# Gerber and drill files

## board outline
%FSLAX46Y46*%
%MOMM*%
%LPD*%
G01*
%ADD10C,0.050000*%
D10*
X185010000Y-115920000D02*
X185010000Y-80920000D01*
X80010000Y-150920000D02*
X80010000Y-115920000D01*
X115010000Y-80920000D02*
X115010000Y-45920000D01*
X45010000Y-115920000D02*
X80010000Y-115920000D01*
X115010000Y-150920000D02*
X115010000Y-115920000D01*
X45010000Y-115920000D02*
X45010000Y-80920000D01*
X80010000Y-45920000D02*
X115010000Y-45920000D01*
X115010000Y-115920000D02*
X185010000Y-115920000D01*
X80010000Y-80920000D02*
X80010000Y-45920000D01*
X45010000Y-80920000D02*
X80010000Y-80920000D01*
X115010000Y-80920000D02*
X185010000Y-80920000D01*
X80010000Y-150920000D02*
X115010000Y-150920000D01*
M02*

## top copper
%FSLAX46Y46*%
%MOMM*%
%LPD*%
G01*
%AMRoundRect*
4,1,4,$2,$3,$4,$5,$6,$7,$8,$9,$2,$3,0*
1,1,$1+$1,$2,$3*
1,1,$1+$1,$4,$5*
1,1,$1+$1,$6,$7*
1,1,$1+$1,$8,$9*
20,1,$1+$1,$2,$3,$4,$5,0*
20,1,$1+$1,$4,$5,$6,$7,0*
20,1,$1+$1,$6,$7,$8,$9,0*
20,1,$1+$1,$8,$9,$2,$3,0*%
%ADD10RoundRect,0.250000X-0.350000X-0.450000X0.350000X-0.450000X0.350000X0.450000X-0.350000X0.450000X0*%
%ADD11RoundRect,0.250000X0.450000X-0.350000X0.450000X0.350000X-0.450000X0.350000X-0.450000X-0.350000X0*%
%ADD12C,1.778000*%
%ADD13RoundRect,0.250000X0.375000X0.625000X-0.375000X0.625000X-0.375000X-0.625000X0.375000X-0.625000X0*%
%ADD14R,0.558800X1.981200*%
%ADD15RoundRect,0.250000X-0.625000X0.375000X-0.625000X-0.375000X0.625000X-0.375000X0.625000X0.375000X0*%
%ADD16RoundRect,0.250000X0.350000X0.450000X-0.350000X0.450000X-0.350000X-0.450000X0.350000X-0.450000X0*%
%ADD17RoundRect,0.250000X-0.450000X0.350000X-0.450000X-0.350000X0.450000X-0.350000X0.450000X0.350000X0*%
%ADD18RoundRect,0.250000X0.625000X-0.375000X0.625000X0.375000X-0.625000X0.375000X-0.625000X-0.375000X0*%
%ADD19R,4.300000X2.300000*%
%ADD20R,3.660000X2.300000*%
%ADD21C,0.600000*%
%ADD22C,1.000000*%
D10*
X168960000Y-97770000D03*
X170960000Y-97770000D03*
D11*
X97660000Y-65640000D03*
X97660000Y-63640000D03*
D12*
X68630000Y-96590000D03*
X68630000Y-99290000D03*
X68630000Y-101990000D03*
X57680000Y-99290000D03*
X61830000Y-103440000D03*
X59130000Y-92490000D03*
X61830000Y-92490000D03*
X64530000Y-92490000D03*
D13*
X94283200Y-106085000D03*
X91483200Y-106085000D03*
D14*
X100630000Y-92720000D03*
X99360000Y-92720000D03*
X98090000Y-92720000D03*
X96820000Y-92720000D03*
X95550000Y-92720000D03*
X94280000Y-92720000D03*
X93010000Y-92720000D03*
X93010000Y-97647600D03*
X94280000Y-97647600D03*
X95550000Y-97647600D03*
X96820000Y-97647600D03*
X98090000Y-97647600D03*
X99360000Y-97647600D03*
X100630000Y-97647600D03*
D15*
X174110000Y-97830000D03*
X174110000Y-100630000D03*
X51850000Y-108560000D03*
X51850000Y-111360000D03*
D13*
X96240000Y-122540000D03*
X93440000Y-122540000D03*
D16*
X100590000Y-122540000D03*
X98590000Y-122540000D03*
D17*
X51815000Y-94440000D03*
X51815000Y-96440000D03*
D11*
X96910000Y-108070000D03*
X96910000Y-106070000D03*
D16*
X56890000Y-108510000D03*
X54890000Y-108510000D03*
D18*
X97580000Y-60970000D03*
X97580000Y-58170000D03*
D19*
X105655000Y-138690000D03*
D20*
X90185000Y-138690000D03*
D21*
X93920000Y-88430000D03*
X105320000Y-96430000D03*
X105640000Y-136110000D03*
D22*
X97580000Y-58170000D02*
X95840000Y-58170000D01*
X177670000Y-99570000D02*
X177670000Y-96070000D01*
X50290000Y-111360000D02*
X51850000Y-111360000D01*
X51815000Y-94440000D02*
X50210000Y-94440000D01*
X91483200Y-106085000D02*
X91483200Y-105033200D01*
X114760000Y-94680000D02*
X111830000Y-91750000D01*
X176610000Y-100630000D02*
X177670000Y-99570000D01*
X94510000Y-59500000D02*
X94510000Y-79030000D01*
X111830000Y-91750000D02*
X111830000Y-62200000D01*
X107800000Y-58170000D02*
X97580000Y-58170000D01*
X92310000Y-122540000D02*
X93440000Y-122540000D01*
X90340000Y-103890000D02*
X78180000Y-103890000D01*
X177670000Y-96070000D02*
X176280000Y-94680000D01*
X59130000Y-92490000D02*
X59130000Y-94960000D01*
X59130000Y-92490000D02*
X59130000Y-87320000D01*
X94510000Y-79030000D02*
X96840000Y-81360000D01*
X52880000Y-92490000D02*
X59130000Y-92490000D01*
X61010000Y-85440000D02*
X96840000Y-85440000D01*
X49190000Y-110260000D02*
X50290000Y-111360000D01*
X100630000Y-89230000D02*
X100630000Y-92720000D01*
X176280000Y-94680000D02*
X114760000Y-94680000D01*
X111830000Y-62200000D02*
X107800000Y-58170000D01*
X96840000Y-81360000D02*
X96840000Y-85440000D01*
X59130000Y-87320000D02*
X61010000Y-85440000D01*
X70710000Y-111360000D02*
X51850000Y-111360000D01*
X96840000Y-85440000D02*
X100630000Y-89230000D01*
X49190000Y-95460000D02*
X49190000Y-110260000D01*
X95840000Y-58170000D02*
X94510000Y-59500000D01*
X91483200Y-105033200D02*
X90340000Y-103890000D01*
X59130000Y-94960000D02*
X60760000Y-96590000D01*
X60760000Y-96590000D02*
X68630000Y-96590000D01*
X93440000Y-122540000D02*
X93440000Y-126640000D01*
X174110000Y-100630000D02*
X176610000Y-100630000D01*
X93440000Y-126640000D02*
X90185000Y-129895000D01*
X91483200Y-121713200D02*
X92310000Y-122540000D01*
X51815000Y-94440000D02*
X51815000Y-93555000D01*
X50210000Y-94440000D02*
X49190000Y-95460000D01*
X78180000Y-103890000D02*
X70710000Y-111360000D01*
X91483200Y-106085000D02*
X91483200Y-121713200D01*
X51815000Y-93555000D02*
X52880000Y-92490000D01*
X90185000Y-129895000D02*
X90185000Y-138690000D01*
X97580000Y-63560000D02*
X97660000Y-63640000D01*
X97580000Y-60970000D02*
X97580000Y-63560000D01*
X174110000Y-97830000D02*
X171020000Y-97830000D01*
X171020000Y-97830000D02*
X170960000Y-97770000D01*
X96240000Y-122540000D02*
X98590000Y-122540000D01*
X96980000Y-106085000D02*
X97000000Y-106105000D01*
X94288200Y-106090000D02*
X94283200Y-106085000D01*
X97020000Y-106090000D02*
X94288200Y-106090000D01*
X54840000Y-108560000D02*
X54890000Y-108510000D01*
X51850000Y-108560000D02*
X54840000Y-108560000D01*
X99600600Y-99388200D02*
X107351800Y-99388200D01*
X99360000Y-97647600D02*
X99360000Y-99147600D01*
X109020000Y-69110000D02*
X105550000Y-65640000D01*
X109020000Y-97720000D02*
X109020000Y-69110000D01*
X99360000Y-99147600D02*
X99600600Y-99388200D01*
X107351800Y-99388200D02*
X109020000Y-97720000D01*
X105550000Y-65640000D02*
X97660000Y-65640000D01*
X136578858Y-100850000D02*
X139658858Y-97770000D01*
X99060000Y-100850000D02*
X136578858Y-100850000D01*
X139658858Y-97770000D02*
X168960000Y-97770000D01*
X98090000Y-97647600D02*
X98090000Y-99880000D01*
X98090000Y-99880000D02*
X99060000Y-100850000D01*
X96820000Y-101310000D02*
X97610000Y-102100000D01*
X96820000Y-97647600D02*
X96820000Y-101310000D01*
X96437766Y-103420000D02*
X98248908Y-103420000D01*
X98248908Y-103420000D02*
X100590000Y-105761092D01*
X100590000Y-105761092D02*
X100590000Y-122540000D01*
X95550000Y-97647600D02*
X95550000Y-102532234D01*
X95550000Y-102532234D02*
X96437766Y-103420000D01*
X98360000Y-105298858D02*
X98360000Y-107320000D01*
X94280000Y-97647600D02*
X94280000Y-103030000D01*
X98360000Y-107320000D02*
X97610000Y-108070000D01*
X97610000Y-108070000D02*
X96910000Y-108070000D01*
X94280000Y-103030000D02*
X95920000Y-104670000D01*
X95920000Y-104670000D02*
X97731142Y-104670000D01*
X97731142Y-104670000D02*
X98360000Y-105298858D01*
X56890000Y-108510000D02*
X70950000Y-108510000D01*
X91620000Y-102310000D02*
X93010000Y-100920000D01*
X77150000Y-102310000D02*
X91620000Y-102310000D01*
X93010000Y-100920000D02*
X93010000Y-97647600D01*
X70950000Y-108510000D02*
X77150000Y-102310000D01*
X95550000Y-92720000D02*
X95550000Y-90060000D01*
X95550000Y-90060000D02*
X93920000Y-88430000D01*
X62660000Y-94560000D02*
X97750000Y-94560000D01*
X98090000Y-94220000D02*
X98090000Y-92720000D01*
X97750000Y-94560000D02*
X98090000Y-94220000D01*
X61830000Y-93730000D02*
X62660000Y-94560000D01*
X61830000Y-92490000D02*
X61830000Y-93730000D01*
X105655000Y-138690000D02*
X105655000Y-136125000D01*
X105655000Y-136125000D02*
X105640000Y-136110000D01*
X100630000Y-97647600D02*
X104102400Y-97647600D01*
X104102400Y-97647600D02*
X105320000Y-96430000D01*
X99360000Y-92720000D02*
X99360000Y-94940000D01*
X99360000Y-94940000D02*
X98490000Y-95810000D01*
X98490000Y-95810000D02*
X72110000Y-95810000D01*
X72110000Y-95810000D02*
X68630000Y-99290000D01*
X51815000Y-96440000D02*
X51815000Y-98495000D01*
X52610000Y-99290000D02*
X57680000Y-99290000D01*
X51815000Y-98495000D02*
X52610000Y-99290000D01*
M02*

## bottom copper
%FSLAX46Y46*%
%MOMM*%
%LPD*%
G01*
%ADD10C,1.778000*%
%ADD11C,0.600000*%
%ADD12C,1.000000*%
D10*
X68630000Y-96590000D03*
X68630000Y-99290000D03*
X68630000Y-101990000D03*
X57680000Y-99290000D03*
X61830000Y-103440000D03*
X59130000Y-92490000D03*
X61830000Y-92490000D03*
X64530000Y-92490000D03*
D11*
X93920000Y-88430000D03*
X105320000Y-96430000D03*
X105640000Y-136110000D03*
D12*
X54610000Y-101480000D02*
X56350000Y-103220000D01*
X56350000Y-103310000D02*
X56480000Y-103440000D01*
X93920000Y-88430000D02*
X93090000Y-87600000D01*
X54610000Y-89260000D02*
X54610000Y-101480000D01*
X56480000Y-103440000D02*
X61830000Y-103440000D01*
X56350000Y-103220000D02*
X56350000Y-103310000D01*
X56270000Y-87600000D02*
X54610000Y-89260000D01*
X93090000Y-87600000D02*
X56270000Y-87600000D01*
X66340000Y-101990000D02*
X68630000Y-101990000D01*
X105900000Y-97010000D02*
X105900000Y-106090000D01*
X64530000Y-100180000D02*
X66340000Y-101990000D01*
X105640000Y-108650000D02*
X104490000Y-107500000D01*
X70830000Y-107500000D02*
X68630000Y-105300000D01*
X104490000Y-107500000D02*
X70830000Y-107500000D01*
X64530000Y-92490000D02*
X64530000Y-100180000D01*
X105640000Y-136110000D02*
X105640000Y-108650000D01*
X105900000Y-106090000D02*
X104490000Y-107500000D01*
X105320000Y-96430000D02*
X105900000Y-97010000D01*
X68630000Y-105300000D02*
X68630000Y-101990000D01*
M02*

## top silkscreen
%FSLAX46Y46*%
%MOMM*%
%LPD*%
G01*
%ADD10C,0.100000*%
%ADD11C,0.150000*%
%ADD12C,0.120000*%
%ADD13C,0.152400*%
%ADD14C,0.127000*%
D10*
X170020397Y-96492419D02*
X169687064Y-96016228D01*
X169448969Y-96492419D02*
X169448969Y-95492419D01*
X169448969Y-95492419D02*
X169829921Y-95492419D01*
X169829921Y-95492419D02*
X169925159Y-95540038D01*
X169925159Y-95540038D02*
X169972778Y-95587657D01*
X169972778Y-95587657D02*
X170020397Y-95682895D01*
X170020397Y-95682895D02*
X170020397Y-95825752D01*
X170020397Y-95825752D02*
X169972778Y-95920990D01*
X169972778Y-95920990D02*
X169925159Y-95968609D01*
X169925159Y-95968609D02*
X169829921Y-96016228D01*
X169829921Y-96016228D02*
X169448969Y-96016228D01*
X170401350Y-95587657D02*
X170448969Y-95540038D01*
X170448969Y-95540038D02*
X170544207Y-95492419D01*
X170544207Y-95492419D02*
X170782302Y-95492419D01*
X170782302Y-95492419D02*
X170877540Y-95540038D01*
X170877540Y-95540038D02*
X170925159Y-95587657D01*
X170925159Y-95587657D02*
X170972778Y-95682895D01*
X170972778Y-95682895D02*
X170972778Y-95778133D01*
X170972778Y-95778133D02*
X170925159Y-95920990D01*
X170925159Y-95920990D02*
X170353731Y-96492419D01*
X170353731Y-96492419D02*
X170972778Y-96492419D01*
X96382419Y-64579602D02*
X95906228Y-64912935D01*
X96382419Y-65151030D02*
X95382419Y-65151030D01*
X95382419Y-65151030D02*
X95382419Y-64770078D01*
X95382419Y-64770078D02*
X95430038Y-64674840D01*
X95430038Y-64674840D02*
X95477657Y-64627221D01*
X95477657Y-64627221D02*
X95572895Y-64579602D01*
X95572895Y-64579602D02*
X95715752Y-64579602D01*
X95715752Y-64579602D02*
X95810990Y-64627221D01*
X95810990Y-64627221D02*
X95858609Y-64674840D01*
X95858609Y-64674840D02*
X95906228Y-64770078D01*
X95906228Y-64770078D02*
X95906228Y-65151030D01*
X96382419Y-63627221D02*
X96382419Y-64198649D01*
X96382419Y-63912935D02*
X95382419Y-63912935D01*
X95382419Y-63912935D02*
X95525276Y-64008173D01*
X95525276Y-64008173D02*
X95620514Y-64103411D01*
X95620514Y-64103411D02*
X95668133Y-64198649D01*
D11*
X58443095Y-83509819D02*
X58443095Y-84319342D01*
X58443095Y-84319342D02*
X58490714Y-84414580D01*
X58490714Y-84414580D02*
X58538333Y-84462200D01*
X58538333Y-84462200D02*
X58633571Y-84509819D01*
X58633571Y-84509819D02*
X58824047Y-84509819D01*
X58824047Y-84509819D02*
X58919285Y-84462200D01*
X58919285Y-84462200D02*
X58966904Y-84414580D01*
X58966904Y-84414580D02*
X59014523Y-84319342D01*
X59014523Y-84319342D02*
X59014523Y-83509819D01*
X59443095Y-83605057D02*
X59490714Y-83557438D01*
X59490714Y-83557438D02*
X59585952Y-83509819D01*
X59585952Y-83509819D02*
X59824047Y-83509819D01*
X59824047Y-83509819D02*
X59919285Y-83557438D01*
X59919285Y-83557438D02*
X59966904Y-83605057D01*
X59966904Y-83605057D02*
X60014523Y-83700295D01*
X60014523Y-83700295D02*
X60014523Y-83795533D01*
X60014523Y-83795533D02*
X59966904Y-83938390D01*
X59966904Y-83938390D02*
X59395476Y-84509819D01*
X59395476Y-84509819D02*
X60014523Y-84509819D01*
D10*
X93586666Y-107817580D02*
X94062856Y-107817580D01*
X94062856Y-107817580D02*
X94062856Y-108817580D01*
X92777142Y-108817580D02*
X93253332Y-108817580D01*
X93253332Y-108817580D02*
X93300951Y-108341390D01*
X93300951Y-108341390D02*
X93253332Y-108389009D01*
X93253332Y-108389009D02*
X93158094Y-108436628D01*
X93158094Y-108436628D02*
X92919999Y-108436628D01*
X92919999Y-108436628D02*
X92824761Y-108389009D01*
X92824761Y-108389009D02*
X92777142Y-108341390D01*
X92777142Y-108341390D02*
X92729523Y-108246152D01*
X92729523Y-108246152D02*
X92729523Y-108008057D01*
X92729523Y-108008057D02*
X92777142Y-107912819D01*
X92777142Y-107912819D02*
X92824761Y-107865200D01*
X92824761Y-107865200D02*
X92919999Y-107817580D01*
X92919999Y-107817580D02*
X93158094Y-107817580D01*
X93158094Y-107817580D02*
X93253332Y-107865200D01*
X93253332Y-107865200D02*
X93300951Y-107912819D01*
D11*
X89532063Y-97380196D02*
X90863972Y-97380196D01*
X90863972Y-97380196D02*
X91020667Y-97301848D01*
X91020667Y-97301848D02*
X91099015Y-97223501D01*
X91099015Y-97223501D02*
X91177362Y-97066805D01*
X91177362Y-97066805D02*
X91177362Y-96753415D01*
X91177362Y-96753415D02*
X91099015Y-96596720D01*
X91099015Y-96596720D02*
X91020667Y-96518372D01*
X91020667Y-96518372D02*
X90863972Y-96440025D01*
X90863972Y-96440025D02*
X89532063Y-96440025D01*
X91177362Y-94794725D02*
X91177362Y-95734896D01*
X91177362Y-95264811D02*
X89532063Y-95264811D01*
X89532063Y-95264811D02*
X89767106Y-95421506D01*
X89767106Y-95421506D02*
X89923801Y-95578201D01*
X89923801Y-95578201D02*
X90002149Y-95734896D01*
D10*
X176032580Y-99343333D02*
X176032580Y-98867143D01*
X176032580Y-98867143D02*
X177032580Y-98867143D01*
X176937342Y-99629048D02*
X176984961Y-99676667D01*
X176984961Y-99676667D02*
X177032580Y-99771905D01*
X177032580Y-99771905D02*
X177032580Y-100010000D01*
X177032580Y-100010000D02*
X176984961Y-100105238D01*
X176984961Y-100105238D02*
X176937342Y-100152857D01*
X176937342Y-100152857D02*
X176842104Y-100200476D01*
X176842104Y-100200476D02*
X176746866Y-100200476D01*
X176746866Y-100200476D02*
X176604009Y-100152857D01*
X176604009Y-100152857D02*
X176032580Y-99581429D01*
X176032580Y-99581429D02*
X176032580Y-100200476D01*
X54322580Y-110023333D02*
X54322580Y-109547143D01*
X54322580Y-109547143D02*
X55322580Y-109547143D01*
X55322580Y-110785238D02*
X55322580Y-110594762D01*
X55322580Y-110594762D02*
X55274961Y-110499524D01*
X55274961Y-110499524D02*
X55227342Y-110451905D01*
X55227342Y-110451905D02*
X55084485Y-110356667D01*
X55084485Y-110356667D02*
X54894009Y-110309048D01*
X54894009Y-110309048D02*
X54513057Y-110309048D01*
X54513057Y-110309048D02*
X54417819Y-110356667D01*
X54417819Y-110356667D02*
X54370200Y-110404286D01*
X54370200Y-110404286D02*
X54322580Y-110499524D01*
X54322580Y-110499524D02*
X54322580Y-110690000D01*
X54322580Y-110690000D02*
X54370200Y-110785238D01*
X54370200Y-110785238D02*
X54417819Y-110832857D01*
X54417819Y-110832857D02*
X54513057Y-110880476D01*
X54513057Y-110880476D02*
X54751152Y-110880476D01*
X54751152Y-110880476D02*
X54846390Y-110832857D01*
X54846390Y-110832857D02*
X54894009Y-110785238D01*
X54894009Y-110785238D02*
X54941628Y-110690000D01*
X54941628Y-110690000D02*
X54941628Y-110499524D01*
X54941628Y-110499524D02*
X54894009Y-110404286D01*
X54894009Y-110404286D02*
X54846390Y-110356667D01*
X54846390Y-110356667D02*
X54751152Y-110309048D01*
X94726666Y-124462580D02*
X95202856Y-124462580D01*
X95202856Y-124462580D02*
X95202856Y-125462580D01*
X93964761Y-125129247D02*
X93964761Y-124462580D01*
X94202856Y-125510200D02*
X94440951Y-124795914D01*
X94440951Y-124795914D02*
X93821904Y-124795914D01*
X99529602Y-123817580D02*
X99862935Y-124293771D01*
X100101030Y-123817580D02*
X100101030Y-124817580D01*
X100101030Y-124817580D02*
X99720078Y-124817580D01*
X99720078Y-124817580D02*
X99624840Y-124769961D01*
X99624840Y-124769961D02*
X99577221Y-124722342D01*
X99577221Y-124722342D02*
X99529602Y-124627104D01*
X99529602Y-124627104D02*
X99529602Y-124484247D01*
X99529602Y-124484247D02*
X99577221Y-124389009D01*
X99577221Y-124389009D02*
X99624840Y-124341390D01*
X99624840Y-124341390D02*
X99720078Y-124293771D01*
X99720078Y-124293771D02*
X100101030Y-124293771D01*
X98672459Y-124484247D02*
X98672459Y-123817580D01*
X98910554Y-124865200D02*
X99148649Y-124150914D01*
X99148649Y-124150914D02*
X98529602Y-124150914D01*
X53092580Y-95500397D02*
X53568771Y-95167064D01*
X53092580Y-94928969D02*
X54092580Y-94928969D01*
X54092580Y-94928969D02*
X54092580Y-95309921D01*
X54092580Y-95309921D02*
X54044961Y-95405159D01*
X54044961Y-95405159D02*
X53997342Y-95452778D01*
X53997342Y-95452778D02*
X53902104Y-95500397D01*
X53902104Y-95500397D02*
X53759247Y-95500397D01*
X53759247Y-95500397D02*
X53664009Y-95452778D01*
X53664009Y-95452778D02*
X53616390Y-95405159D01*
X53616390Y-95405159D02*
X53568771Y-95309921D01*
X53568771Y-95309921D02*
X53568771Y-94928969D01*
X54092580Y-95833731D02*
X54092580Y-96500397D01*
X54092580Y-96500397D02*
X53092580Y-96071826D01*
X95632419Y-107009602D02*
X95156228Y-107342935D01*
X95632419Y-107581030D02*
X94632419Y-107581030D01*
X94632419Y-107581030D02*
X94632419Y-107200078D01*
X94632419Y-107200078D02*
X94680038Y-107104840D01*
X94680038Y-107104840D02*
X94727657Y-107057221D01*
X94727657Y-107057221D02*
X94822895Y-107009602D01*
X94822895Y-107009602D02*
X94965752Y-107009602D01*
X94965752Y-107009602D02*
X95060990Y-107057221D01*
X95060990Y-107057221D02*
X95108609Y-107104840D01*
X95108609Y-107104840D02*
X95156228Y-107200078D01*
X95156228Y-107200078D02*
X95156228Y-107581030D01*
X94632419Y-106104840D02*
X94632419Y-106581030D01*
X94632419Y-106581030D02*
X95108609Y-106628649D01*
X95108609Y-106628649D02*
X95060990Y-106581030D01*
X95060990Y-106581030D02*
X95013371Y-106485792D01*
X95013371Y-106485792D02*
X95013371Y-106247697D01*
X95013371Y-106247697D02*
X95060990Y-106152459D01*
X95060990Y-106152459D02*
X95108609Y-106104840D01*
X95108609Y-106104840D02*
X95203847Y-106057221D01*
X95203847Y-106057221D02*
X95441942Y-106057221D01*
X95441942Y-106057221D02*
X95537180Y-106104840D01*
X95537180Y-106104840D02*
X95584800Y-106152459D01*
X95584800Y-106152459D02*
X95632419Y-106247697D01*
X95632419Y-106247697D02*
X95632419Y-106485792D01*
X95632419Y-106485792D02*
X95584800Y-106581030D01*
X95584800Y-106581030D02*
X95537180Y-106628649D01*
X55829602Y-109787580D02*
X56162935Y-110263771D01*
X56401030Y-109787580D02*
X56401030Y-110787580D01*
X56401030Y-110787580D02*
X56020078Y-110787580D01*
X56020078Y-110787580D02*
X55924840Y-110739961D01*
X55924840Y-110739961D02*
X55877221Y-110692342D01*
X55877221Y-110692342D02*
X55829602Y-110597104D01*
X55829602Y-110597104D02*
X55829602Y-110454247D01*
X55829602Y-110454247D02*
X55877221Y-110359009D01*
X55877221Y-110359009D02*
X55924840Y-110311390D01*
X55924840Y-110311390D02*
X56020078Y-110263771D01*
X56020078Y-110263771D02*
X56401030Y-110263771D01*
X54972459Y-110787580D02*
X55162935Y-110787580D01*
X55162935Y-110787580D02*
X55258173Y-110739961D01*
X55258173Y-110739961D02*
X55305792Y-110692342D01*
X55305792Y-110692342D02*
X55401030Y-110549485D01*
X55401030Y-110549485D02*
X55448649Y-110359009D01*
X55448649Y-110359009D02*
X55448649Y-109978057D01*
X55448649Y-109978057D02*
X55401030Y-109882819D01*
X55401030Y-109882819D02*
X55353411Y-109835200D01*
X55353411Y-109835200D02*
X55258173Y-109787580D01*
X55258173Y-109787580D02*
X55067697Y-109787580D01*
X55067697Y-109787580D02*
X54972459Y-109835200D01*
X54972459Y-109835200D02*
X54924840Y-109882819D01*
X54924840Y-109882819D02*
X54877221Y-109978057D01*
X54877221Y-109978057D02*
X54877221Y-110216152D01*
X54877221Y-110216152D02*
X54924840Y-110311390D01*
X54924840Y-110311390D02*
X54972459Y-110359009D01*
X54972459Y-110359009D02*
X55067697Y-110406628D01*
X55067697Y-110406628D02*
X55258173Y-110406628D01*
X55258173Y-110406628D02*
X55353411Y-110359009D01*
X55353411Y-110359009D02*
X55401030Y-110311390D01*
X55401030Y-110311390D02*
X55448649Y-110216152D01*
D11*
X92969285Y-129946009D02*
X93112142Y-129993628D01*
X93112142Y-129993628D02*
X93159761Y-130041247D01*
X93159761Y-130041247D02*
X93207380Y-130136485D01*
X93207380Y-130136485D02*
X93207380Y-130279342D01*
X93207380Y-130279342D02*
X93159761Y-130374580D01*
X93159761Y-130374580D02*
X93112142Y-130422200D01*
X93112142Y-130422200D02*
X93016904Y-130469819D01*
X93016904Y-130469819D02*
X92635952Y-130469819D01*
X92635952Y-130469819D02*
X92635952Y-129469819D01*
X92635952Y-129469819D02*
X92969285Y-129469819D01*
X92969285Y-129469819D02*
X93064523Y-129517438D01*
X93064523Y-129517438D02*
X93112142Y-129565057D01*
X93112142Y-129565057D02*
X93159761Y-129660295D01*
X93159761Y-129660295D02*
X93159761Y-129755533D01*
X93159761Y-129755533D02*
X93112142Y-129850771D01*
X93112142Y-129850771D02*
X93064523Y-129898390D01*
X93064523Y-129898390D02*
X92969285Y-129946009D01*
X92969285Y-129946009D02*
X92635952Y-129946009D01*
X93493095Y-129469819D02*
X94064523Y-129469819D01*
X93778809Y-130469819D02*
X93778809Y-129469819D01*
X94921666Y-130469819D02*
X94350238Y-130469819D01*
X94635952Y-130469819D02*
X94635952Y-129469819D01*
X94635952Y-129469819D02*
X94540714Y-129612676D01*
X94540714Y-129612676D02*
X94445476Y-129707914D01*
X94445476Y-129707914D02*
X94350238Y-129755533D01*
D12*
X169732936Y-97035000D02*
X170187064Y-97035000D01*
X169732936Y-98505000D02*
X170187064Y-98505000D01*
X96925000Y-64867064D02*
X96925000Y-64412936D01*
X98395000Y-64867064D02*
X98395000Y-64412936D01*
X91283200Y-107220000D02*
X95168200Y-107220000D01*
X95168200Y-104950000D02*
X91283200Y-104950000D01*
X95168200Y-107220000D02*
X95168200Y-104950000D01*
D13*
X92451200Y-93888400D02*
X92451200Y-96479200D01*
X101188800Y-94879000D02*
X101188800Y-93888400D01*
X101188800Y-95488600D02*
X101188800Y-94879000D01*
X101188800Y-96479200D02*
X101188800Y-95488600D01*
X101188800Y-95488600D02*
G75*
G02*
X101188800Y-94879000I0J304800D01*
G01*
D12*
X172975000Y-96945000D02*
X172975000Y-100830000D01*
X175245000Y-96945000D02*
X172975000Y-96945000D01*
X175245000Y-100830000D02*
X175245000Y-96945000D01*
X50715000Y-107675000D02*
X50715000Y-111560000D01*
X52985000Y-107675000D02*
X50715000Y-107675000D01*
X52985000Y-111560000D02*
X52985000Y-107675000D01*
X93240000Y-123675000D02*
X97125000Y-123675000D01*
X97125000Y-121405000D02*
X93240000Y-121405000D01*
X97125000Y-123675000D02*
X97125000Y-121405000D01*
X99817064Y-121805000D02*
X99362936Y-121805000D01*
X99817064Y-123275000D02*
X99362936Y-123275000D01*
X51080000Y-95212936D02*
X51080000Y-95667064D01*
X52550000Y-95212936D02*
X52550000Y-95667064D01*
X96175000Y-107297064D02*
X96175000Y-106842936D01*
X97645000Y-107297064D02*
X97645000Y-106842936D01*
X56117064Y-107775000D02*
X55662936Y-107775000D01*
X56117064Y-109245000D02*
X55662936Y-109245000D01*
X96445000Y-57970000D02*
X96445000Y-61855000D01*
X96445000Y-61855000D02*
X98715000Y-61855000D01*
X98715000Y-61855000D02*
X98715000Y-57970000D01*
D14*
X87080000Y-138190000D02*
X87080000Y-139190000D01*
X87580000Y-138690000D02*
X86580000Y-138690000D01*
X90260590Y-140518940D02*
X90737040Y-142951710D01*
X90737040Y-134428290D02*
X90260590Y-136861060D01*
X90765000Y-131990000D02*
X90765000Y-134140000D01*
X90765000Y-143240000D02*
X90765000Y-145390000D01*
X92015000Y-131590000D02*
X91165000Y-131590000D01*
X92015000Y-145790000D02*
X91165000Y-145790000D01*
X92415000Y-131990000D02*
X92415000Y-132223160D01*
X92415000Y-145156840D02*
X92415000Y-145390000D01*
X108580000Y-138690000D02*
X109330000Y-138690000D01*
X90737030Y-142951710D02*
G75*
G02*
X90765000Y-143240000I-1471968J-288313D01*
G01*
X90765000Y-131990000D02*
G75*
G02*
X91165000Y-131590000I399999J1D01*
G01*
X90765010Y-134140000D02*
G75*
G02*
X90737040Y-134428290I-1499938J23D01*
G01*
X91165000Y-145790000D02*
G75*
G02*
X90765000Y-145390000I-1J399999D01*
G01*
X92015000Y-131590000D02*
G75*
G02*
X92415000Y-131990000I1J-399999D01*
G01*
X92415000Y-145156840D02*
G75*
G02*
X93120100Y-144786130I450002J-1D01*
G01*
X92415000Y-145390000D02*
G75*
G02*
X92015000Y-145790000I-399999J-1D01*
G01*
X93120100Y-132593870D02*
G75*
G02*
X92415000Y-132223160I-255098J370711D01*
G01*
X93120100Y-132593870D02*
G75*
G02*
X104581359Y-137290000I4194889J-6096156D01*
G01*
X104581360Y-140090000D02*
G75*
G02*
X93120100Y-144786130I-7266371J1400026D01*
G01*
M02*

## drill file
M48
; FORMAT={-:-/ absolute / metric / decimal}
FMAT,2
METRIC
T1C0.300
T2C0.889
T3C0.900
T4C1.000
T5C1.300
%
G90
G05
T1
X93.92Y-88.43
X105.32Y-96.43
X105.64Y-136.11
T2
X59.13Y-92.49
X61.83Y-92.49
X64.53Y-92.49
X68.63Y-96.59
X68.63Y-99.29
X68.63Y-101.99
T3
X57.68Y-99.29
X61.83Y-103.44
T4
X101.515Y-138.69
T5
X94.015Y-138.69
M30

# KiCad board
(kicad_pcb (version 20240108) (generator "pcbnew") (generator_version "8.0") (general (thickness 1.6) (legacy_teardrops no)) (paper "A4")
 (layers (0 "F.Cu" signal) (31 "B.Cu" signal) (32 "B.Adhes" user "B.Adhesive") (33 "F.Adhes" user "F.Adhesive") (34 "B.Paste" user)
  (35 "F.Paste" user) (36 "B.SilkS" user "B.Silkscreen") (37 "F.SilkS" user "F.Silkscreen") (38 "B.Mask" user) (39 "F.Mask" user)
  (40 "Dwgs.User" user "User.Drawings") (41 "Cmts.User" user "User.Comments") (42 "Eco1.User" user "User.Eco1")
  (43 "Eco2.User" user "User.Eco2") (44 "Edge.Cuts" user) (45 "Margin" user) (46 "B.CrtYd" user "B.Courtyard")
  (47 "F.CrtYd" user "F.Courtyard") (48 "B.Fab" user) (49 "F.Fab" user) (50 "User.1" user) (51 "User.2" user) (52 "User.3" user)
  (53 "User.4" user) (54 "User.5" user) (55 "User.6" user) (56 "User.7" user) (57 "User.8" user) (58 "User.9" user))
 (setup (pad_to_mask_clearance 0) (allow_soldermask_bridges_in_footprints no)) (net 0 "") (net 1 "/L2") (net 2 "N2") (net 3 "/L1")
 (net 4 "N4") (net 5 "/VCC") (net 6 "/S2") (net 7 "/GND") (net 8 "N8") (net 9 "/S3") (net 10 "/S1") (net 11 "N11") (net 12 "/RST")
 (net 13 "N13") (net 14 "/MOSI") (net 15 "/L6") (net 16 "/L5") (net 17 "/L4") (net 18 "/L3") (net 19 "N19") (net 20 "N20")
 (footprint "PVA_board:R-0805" (layer "F.Cu") (at 169.96 97.755)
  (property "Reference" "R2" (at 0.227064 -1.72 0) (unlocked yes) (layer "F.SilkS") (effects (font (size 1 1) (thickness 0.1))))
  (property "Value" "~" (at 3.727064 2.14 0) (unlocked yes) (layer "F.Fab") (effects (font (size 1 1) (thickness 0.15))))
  (fp_line (start -0.227064 -0.72) (end 0.227064 -0.72) (stroke (width 0.12) (type solid)) (layer "F.SilkS"))
  (fp_line (start -0.227064 0.75) (end 0.227064 0.75) (stroke (width 0.12) (type solid)) (layer "F.SilkS"))
  (pad "1" smd roundrect (at -1 0.015) (size 1.2 1.4) (layers "F.Cu" "F.Paste" "F.Mask") (roundrect_rratio 0.208333) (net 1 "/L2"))
  (pad "2" smd roundrect (at 1 0.015) (size 1.2 1.4) (layers "F.Cu" "F.Paste" "F.Mask") (roundrect_rratio 0.208333) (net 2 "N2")))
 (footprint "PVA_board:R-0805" (layer "F.Cu") (at 97.645 64.64 90)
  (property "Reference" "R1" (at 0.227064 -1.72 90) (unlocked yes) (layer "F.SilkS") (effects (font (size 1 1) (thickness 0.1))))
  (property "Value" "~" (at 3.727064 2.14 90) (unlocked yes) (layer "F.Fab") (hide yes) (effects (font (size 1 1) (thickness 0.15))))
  (fp_line (start -0.227064 -0.72) (end 0.227064 -0.72) (stroke (width 0.12) (type solid)) (layer "F.SilkS"))
  (fp_line (start -0.227064 0.75) (end 0.227064 0.75) (stroke (width 0.12) (type solid)) (layer "F.SilkS"))
  (pad "1" smd roundrect (at -1 0.015 90) (size 1.2 1.4) (layers "F.Cu" "F.Paste" "F.Mask") (roundrect_rratio 0.208333) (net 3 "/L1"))
  (pad "2" smd roundrect (at 1 0.015 90) (size 1.2 1.4) (layers "F.Cu" "F.Paste" "F.Mask") (roundrect_rratio 0.208333) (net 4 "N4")))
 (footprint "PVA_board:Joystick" (layer "F.Cu") (at 61.83 99.29)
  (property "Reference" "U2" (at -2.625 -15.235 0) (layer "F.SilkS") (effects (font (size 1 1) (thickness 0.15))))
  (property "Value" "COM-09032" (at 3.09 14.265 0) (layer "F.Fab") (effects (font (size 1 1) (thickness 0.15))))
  (pad "H1" thru_hole circle (at 6.8 -2.7) (size 1.778 1.778) (drill 0.889) (layers "*.Cu" "*.Mask") (remove_unused_layers no)
   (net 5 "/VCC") (solder_mask_margin 0.102))
  (pad "H2" thru_hole circle (at 6.8 0) (size 1.778 1.778) (drill 0.889) (layers "*.Cu" "*.Mask") (remove_unused_layers no) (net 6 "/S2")
   (solder_mask_margin 0.102))
  (pad "H3" thru_hole circle (at 6.8 2.7) (size 1.778 1.778) (drill 0.889) (layers "*.Cu" "*.Mask") (remove_unused_layers no) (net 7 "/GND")
   (solder_mask_margin 0.102))
  (pad "Sa" thru_hole circle (at -4.15 0) (size 1.778 1.778) (drill 0.9) (layers "*.Cu" "*.Mask") (remove_unused_layers no) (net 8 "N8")
   (solder_mask_margin 0.102))
  (pad "Sb" thru_hole circle (at 0 4.15) (size 1.778 1.778) (drill 0.9) (layers "*.Cu" "*.Mask") (remove_unused_layers no) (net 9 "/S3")
   (solder_mask_margin 0.102))
  (pad "V1" thru_hole circle (at -2.7 -6.8) (size 1.778 1.778) (drill 0.889) (layers "*.Cu" "*.Mask") (remove_unused_layers no)
   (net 5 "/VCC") (solder_mask_margin 0.102))
  (pad "V2" thru_hole circle (at 0 -6.8) (size 1.778 1.778) (drill 0.889) (layers "*.Cu" "*.Mask") (remove_unused_layers no) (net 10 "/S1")
   (solder_mask_margin 0.102))
  (pad "V3" thru_hole circle (at 2.7 -6.8) (size 1.778 1.778) (drill 0.889) (layers "*.Cu" "*.Mask") (remove_unused_layers no)
   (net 7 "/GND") (solder_mask_margin 0.102)))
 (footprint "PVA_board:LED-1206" (layer "F.Cu") (at 92.8832 106.085 180)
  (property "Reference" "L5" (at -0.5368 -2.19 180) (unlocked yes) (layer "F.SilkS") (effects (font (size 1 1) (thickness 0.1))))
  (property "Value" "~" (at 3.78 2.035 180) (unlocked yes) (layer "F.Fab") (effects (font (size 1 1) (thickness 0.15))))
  (fp_line (start 1.6 -1.135) (end -2.285 -1.135) (stroke (width 0.12) (type solid)) (layer "F.SilkS"))
  (fp_line (start -2.285 1.135) (end 1.6 1.135) (stroke (width 0.12) (type solid)) (layer "F.SilkS"))
  (fp_line (start -2.285 -1.135) (end -2.285 1.135) (stroke (width 0.12) (type solid)) (layer "F.SilkS"))
  (pad "1" smd roundrect (at -1.4 0 180) (size 1.25 1.75) (layers "F.Cu" "F.Paste" "F.Mask") (roundrect_rratio 0.2) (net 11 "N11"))
  (pad "2" smd roundrect (at 1.4 0 180) (size 1.25 1.75) (layers "F.Cu" "F.Paste" "F.Mask") (roundrect_rratio 0.2) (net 5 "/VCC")))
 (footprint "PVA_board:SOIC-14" (layer "F.Cu") (at 96.82 95.1838 -90)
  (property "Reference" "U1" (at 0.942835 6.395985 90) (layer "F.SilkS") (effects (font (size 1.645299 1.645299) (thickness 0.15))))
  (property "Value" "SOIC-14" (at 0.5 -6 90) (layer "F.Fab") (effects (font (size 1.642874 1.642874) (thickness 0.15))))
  (fp_line (start -1.2954 4.3688) (end 1.2954 4.3688) (stroke (width 0.1524) (type solid)) (layer "F.SilkS"))
  (fp_line (start -0.3048 -4.3688) (end -1.2954 -4.3688) (stroke (width 0.1524) (type solid)) (layer "F.SilkS"))
  (fp_line (start 0.3048 -4.3688) (end -0.3048 -4.3688) (stroke (width 0.1524) (type solid)) (layer "F.SilkS"))
  (fp_line (start 1.2954 -4.3688) (end 0.3048 -4.3688) (stroke (width 0.1524) (type solid)) (layer "F.SilkS"))
  (fp_arc (start 0.3048 -4.3688) (mid 0 -4.064) (end -0.3048 -4.3688) (stroke (width 0.1524) (type solid)) (layer "F.SilkS"))
  (pad "1" smd rect (at -2.4638 -3.81 270) (size 1.9812 0.5588) (layers "F.Cu" "F.Paste" "F.Mask") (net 5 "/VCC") (solder_mask_margin 0.102))
  (pad "2" smd rect (at -2.4638 -2.54 270) (size 1.9812 0.5588) (layers "F.Cu" "F.Paste" "F.Mask") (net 6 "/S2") (solder_mask_margin 0.102))
  (pad "3" smd rect (at -2.4638 -1.27 270) (size 1.9812 0.5588) (layers "F.Cu" "F.Paste" "F.Mask") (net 10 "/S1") (solder_mask_margin 0.102))
  (pad "4" smd rect (at -2.4638 0 270) (size 1.9812 0.5588) (layers "F.Cu" "F.Paste" "F.Mask") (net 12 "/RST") (solder_mask_margin 0.102))
  (pad "5" smd rect (at -2.4638 1.27 270) (size 1.9812 0.5588) (layers "F.Cu" "F.Paste" "F.Mask") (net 9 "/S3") (solder_mask_margin 0.102))
  (pad "6" smd rect (at -2.4638 2.54 270) (size 1.9812 0.5588) (layers "F.Cu" "F.Paste" "F.Mask") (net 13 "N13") (solder_mask_margin 0.102))
  (pad "7" smd rect (at -2.4638 3.81 270) (size 1.9812 0.5588) (layers "F.Cu" "F.Paste" "F.Mask") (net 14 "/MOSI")
   (solder_mask_margin 0.102))
  (pad "8" smd rect (at 2.4638 3.81 270) (size 1.9812 0.5588) (layers "F.Cu" "F.Paste" "F.Mask") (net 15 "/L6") (solder_mask_margin 0.102))
  (pad "9" smd rect (at 2.4638 2.54 270) (size 1.9812 0.5588) (layers "F.Cu" "F.Paste" "F.Mask") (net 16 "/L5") (solder_mask_margin 0.102))
  (pad "10" smd rect (at 2.4638 1.27 270) (size 1.9812 0.5588) (layers "F.Cu" "F.Paste" "F.Mask") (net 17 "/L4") (solder_mask_margin 0.102))
  (pad "11" smd rect (at 2.4638 0 270) (size 1.9812 0.5588) (layers "F.Cu" "F.Paste" "F.Mask") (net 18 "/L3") (solder_mask_margin 0.102))
  (pad "12" smd rect (at 2.4638 -1.27 270) (size 1.9812 0.5588) (layers "F.Cu" "F.Paste" "F.Mask") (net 1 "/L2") (solder_mask_margin 0.102))
  (pad "13" smd rect (at 2.4638 -2.54 270) (size 1.9812 0.5588) (layers "F.Cu" "F.Paste" "F.Mask") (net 3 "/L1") (solder_mask_margin 0.102))
  (pad "14" smd rect (at 2.4638 -3.81 270) (size 1.9812 0.5588) (layers "F.Cu" "F.Paste" "F.Mask") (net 7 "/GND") (solder_mask_margin 0.102)))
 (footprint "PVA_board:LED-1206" (layer "F.Cu") (at 174.11 99.23 -90)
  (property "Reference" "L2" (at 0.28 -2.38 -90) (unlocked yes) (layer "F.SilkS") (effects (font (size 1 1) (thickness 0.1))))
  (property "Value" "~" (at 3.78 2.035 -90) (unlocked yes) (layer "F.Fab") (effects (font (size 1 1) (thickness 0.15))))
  (fp_line (start -2.285 1.135) (end 1.6 1.135) (stroke (width 0.12) (type solid)) (layer "F.SilkS"))
  (fp_line (start -2.285 -1.135) (end -2.285 1.135) (stroke (width 0.12) (type solid)) (layer "F.SilkS"))
  (fp_line (start 1.6 -1.135) (end -2.285 -1.135) (stroke (width 0.12) (type solid)) (layer "F.SilkS"))
  (pad "1" smd roundrect (at -1.4 0 270) (size 1.25 1.75) (layers "F.Cu" "F.Paste" "F.Mask") (roundrect_rratio 0.2) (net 2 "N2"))
  (pad "2" smd roundrect (at 1.4 0 270) (size 1.25 1.75) (layers "F.Cu" "F.Paste" "F.Mask") (roundrect_rratio 0.2) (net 5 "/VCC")))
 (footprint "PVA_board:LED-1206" (layer "F.Cu") (at 51.85 109.96 -90)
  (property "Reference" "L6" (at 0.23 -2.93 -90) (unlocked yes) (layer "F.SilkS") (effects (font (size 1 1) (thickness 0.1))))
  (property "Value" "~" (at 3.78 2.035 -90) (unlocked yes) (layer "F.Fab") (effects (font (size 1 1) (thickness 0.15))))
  (fp_line (start -2.285 1.135) (end 1.6 1.135) (stroke (width 0.12) (type solid)) (layer "F.SilkS"))
  (fp_line (start -2.285 -1.135) (end -2.285 1.135) (stroke (width 0.12) (type solid)) (layer "F.SilkS"))
  (fp_line (start 1.6 -1.135) (end -2.285 -1.135) (stroke (width 0.12) (type solid)) (layer "F.SilkS"))
  (pad "1" smd roundrect (at -1.4 0 270) (size 1.25 1.75) (layers "F.Cu" "F.Paste" "F.Mask") (roundrect_rratio 0.2) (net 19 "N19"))
  (pad "2" smd roundrect (at 1.4 0 270) (size 1.25 1.75) (layers "F.Cu" "F.Paste" "F.Mask") (roundrect_rratio 0.2) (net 5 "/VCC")))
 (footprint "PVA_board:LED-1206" (layer "F.Cu") (at 94.84 122.54 180)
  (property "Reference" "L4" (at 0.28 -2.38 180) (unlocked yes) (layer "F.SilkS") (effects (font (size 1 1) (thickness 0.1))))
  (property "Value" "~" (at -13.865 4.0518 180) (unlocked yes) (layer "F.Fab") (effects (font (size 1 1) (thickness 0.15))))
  (fp_line (start 1.6 -1.135) (end -2.285 -1.135) (stroke (width 0.12) (type solid)) (layer "F.SilkS"))
  (fp_line (start -2.285 1.135) (end 1.6 1.135) (stroke (width 0.12) (type solid)) (layer "F.SilkS"))
  (fp_line (start -2.285 -1.135) (end -2.285 1.135) (stroke (width 0.12) (type solid)) (layer "F.SilkS"))
  (pad "1" smd roundrect (at -1.4 0 180) (size 1.25 1.75) (layers "F.Cu" "F.Paste" "F.Mask") (roundrect_rratio 0.2) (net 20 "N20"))
  (pad "2" smd roundrect (at 1.4 0 180) (size 1.25 1.75) (layers "F.Cu" "F.Paste" "F.Mask") (roundrect_rratio 0.2) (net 5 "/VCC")))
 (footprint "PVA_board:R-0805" (layer "F.Cu") (at 99.59 122.555 180)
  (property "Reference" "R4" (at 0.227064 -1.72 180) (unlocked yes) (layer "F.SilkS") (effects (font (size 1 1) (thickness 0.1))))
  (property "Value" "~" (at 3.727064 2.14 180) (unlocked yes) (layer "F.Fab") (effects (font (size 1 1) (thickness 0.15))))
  (fp_line (start -0.227064 0.75) (end 0.227064 0.75) (stroke (width 0.12) (type solid)) (layer "F.SilkS"))
  (fp_line (start -0.227064 -0.72) (end 0.227064 -0.72) (stroke (width 0.12) (type solid)) (layer "F.SilkS"))
  (pad "1" smd roundrect (at -1 0.015 180) (size 1.2 1.4) (layers "F.Cu" "F.Paste" "F.Mask") (roundrect_rratio 0.208333) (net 17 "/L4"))
  (pad "2" smd roundrect (at 1 0.015 180) (size 1.2 1.4) (layers "F.Cu" "F.Paste" "F.Mask") (roundrect_rratio 0.208333) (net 20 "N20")))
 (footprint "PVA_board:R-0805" (layer "F.Cu") (at 51.83 95.44 -90)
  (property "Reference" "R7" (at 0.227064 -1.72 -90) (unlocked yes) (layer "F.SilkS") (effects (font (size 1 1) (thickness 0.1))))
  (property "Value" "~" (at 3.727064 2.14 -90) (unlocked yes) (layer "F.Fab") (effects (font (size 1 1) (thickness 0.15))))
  (fp_line (start -0.227064 0.75) (end 0.227064 0.75) (stroke (width 0.12) (type solid)) (layer "F.SilkS"))
  (fp_line (start -0.227064 -0.72) (end 0.227064 -0.72) (stroke (width 0.12) (type solid)) (layer "F.SilkS"))
  (pad "1" smd roundrect (at -1 0.015 270) (size 1.2 1.4) (layers "F.Cu" "F.Paste" "F.Mask") (roundrect_rratio 0.208333) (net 5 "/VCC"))
  (pad "2" smd roundrect (at 1 0.015 270) (size 1.2 1.4) (layers "F.Cu" "F.Paste" "F.Mask") (roundrect_rratio 0.208333) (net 8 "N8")))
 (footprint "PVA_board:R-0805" (layer "F.Cu") (at 96.895 107.07 90)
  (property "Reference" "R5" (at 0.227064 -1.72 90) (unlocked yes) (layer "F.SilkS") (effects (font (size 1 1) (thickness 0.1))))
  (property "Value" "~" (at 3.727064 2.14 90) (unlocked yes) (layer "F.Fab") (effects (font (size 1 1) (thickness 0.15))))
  (fp_line (start -0.227064 -0.72) (end 0.227064 -0.72) (stroke (width 0.12) (type solid)) (layer "F.SilkS"))
  (fp_line (start -0.227064 0.75) (end 0.227064 0.75) (stroke (width 0.12) (type solid)) (layer "F.SilkS"))
  (pad "1" smd roundrect (at -1 0.015 90) (size 1.2 1.4) (layers "F.Cu" "F.Paste" "F.Mask") (roundrect_rratio 0.208333) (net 16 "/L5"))
  (pad "2" smd roundrect (at 1 0.015 90) (size 1.2 1.4) (layers "F.Cu" "F.Paste" "F.Mask") (roundrect_rratio 0.208333) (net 11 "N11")))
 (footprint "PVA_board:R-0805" (layer "F.Cu") (at 55.89 108.525 180)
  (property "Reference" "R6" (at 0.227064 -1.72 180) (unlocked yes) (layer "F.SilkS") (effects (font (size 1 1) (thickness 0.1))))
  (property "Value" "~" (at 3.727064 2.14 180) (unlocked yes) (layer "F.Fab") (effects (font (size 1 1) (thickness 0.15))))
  (fp_line (start -0.227064 0.75) (end 0.227064 0.75) (stroke (width 0.12) (type solid)) (layer "F.SilkS"))
  (fp_line (start -0.227064 -0.72) (end 0.227064 -0.72) (stroke (width 0.12) (type solid)) (layer "F.SilkS"))
  (pad "1" smd roundrect (at -1 0.015 180) (size 1.2 1.4) (layers "F.Cu" "F.Paste" "F.Mask") (roundrect_rratio 0.208333) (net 15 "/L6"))
  (pad "2" smd roundrect (at 1 0.015 180) (size 1.2 1.4) (layers "F.Cu" "F.Paste" "F.Mask") (roundrect_rratio 0.208333) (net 19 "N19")))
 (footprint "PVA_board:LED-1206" (layer "F.Cu") (at 97.58 59.57 90)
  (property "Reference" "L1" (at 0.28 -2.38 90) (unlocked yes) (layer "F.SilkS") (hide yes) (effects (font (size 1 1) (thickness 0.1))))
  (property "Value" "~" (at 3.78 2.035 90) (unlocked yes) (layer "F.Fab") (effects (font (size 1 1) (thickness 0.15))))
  (fp_line (start 1.6 -1.135) (end -2.285 -1.135) (stroke (width 0.12) (type solid)) (layer "F.SilkS"))
  (fp_line (start -2.285 -1.135) (end -2.285 1.135) (stroke (width 0.12) (type solid)) (layer "F.SilkS"))
  (fp_line (start -2.285 1.135) (end 1.6 1.135) (stroke (width 0.12) (type solid)) (layer "F.SilkS"))
  (pad "1" smd roundrect (at -1.4 0 90) (size 1.25 1.75) (layers "F.Cu" "F.Paste" "F.Mask") (roundrect_rratio 0.2) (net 4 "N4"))
  (pad "2" smd roundrect (at 1.4 0 90) (size 1.25 1.75) (layers "F.Cu" "F.Paste" "F.Mask") (roundrect_rratio 0.2) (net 5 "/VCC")))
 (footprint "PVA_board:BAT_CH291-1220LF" (layer "F.Cu") (at 98.08 138.69)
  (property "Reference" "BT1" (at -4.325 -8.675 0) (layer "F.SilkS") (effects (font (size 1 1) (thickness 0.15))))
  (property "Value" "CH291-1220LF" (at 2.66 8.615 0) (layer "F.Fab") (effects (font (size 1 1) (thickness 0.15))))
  (fp_line (start -11 -0.5) (end -11 0.5) (stroke (width 0.127) (type solid)) (layer "F.SilkS"))
  (fp_line (start -10.5 0) (end -11.5 0) (stroke (width 0.127) (type solid)) (layer "F.SilkS"))
  (fp_line (start -7.81941 1.82894) (end -7.34296 4.26171) (stroke (width 0.127) (type solid)) (layer "F.SilkS"))
  (fp_line (start -7.34296 -4.26171) (end -7.81941 -1.82894) (stroke (width 0.127) (type solid)) (layer "F.SilkS"))
  (fp_line (start -7.315 -6.7) (end -7.315 -4.55) (stroke (width 0.127) (type solid)) (layer "F.SilkS"))
  (fp_line (start -7.315 4.55) (end -7.315 6.7) (stroke (width 0.127) (type solid)) (layer "F.SilkS"))
  (fp_line (start -6.065 -7.1) (end -6.915 -7.1) (stroke (width 0.127) (type solid)) (layer "F.SilkS"))
  (fp_line (start -6.065 7.1) (end -6.915 7.1) (stroke (width 0.127) (type solid)) (layer "F.SilkS"))
  (fp_line (start -5.665 -6.7) (end -5.665 -6.46684) (stroke (width 0.127) (type solid)) (layer "F.SilkS"))
  (fp_line (start -5.665 6.46684) (end -5.665 6.7) (stroke (width 0.127) (type solid)) (layer "F.SilkS"))
  (fp_line (start 10.5 0) (end 11.25 0) (stroke (width 0.127) (type solid)) (layer "F.SilkS"))
  (fp_arc (start -7.34297 4.26171) (mid -7.32201 4.405178) (end -7.315 4.55) (stroke (width 0.127) (type solid)) (layer "F.SilkS"))
  (fp_arc (start -7.315 -6.7) (mid -7.197843 -6.982843) (end -6.915 -7.1) (stroke (width 0.127) (type solid)) (layer "F.SilkS"))
  (fp_arc (start -7.31499 -4.55) (mid -7.322 -4.405178) (end -7.34296 -4.26171) (stroke (width 0.127) (type solid)) (layer "F.SilkS"))
  (fp_arc (start -6.915 7.1) (mid -7.197843 6.982843) (end -7.315 6.7) (stroke (width 0.127) (type solid)) (layer "F.SilkS"))
  (fp_arc (start -6.065 -7.1) (mid -5.782157 -6.982843) (end -5.665 -6.7) (stroke (width 0.127) (type solid)) (layer "F.SilkS"))
  (fp_arc (start -5.665 6.46684) (mid -5.42441 6.068534) (end -4.9599 6.09613) (stroke (width 0.127) (type solid)) (layer "F.SilkS"))
  (fp_arc (start -5.665 6.7) (mid -5.782157 6.982843) (end -6.065 7.1) (stroke (width 0.127) (type solid)) (layer "F.SilkS"))
  (fp_arc (start -4.9599 -6.09613) (mid -5.42441 -6.068534) (end -5.665 -6.46684) (stroke (width 0.127) (type solid)) (layer "F.SilkS"))
  (fp_arc (start -4.9599 -6.09613) (mid 2.040681 -6.847477) (end 6.501359 -1.4) (stroke (width 0.127) (type solid)) (layer "F.SilkS"))
  (fp_arc (start 6.50136 1.4) (mid 2.040681 6.847478) (end -4.9599 6.09613) (stroke (width 0.127) (type solid)) (layer "F.SilkS"))
  (pad "" np_thru_hole circle (at -4.065 0) (size 1.3 1.3) (drill 1.3) (layers "*.Cu" "*.Mask"))
  (pad "" np_thru_hole circle (at 3.435 0) (size 1 1) (drill 1) (layers "*.Cu" "*.Mask"))
  (pad "N" smd rect (at 7.575 0) (size 4.3 2.3) (layers "F.Cu" "F.Paste" "F.Mask") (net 7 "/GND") (solder_mask_margin 0.102))
  (pad "P" smd rect (at -7.895 0) (size 3.66 2.3) (layers "F.Cu" "F.Paste" "F.Mask") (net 5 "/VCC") (solder_mask_margin 0.102)))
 (gr_line (start 185.01 115.92) (end 185.01 80.92) (stroke (width 0.05) (type default)) (layer "Edge.Cuts"))
 (gr_line (start 80.01 150.92) (end 80.01 115.92) (stroke (width 0.05) (type default)) (layer "Edge.Cuts"))
 (gr_line (start 115.01 80.92) (end 115.01 45.92) (stroke (width 0.05) (type default)) (layer "Edge.Cuts"))
 (gr_line (start 45.01 115.92) (end 80.01 115.92) (stroke (width 0.05) (type default)) (layer "Edge.Cuts"))
 (gr_line (start 115.01 150.92) (end 115.01 115.92) (stroke (width 0.05) (type default)) (layer "Edge.Cuts"))
 (gr_line (start 45.01 115.92) (end 45.01 80.92) (stroke (width 0.05) (type default)) (layer "Edge.Cuts"))
 (gr_line (start 80.01 45.92) (end 115.01 45.92) (stroke (width 0.05) (type default)) (layer "Edge.Cuts"))
 (gr_line (start 115.01 115.92) (end 185.01 115.92) (stroke (width 0.05) (type default)) (layer "Edge.Cuts"))
 (gr_line (start 80.01 80.92) (end 80.01 45.92) (stroke (width 0.05) (type default)) (layer "Edge.Cuts"))
 (gr_line (start 45.01 80.92) (end 80.01 80.92) (stroke (width 0.05) (type default)) (layer "Edge.Cuts"))
 (gr_line (start 115.01 80.92) (end 185.01 80.92) (stroke (width 0.05) (type default)) (layer "Edge.Cuts"))
 (gr_line (start 80.01 150.92) (end 115.01 150.92) (stroke (width 0.05) (type default)) (layer "Edge.Cuts"))
 (segment (start 97.58 58.17) (end 95.84 58.17) (width 1) (layer "F.Cu") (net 5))
 (segment (start 177.67 99.57) (end 177.67 96.07) (width 1) (layer "F.Cu") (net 5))
 (segment (start 50.29 111.36) (end 51.85 111.36) (width 1) (layer "F.Cu") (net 5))
 (segment (start 51.815 94.44) (end 50.21 94.44) (width 1) (layer "F.Cu") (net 5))
 (segment (start 91.4832 106.085) (end 91.4832 105.0332) (width 1) (layer "F.Cu") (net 5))
 (segment (start 114.76 94.68) (end 111.83 91.75) (width 1) (layer "F.Cu") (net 5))
 (segment (start 176.61 100.63) (end 177.67 99.57) (width 1) (layer "F.Cu") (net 5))
 (segment (start 94.51 59.5) (end 94.51 79.03) (width 1) (layer "F.Cu") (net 5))
 (segment (start 111.83 91.75) (end 111.83 62.2) (width 1) (layer "F.Cu") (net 5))
 (segment (start 107.8 58.17) (end 97.58 58.17) (width 1) (layer "F.Cu") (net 5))
 (segment (start 92.31 122.54) (end 93.44 122.54) (width 1) (layer "F.Cu") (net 5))
 (segment (start 90.34 103.89) (end 78.18 103.89) (width 1) (layer "F.Cu") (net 5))
 (segment (start 177.67 96.07) (end 176.28 94.68) (width 1) (layer "F.Cu") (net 5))
 (segment (start 59.13 92.49) (end 59.13 94.96) (width 1) (layer "F.Cu") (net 5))
 (segment (start 59.13 92.49) (end 59.13 87.32) (width 1) (layer "F.Cu") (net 5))
 (segment (start 94.51 79.03) (end 96.84 81.36) (width 1) (layer "F.Cu") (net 5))
 (segment (start 52.88 92.49) (end 59.13 92.49) (width 1) (layer "F.Cu") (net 5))
 (segment (start 61.01 85.44) (end 96.84 85.44) (width 1) (layer "F.Cu") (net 5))
 (segment (start 49.19 110.26) (end 50.29 111.36) (width 1) (layer "F.Cu") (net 5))
 (segment (start 100.63 89.23) (end 100.63 92.72) (width 1) (layer "F.Cu") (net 5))
 (segment (start 176.28 94.68) (end 114.76 94.68) (width 1) (layer "F.Cu") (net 5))
 (segment (start 111.83 62.2) (end 107.8 58.17) (width 1) (layer "F.Cu") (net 5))
 (segment (start 96.84 81.36) (end 96.84 85.44) (width 1) (layer "F.Cu") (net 5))
 (segment (start 59.13 87.32) (end 61.01 85.44) (width 1) (layer "F.Cu") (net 5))
 (segment (start 70.71 111.36) (end 51.85 111.36) (width 1) (layer "F.Cu") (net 5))
 (segment (start 96.84 85.44) (end 100.63 89.23) (width 1) (layer "F.Cu") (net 5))
 (segment (start 49.19 95.46) (end 49.19 110.26) (width 1) (layer "F.Cu") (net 5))
 (segment (start 95.84 58.17) (end 94.51 59.5) (width 1) (layer "F.Cu") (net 5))
 (segment (start 91.4832 105.0332) (end 90.34 103.89) (width 1) (layer "F.Cu") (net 5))
 (segment (start 59.13 94.96) (end 60.76 96.59) (width 1) (layer "F.Cu") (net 5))
 (segment (start 60.76 96.59) (end 68.63 96.59) (width 1) (layer "F.Cu") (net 5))
 (segment (start 93.44 122.54) (end 93.44 126.64) (width 1) (layer "F.Cu") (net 5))
 (segment (start 174.11 100.63) (end 176.61 100.63) (width 1) (layer "F.Cu") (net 5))
 (segment (start 93.44 126.64) (end 90.185 129.895) (width 1) (layer "F.Cu") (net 5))
 (segment (start 91.4832 121.7132) (end 92.31 122.54) (width 1) (layer "F.Cu") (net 5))
 (segment (start 51.815 94.44) (end 51.815 93.555) (width 1) (layer "F.Cu") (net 5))
 (segment (start 50.21 94.44) (end 49.19 95.46) (width 1) (layer "F.Cu") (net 5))
 (segment (start 78.18 103.89) (end 70.71 111.36) (width 1) (layer "F.Cu") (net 5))
 (segment (start 91.4832 106.085) (end 91.4832 121.7132) (width 1) (layer "F.Cu") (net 5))
 (segment (start 51.815 93.555) (end 52.88 92.49) (width 1) (layer "F.Cu") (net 5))
 (segment (start 90.185 129.895) (end 90.185 138.69) (width 1) (layer "F.Cu") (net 5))
 (segment (start 97.58 63.56) (end 97.66 63.64) (width 1) (layer "F.Cu") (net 4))
 (segment (start 97.58 60.97) (end 97.58 63.56) (width 1) (layer "F.Cu") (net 4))
 (segment (start 174.11 97.83) (end 171.02 97.83) (width 1) (layer "F.Cu") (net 2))
 (segment (start 171.02 97.83) (end 170.96 97.77) (width 1) (layer "F.Cu") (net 2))
 (segment (start 96.24 122.54) (end 98.59 122.54) (width 1) (layer "F.Cu") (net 20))
 (segment (start 96.98 106.085) (end 97 106.105) (width 1) (layer "F.Cu") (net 11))
 (segment (start 94.2882 106.09) (end 94.2832 106.085) (width 1) (layer "F.Cu") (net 11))
 (segment (start 97.02 106.09) (end 94.2882 106.09) (width 1) (layer "F.Cu") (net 11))
 (segment (start 54.84 108.56) (end 54.89 108.51) (width 1) (layer "F.Cu") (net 19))
 (segment (start 51.85 108.56) (end 54.84 108.56) (width 1) (layer "F.Cu") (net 19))
 (segment (start 99.6006 99.3882) (end 107.3518 99.3882) (width 1) (layer "F.Cu") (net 3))
 (segment (start 99.36 97.6476) (end 99.36 99.1476) (width 1) (layer "F.Cu") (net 3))
 (segment (start 109.02 69.11) (end 105.55 65.64) (width 1) (layer "F.Cu") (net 3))
 (segment (start 109.02 97.72) (end 109.02 69.11) (width 1) (layer "F.Cu") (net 3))
 (segment (start 99.36 99.1476) (end 99.6006 99.3882) (width 1) (layer "F.Cu") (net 3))
 (segment (start 107.3518 99.3882) (end 109.02 97.72) (width 1) (layer "F.Cu") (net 3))
 (segment (start 105.55 65.64) (end 97.66 65.64) (width 1) (layer "F.Cu") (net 3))
 (segment (start 136.578858 100.85) (end 139.658858 97.77) (width 1) (layer "F.Cu") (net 1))
 (segment (start 99.06 100.85) (end 136.578858 100.85) (width 1) (layer "F.Cu") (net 1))
 (segment (start 139.658858 97.77) (end 168.96 97.77) (width 1) (layer "F.Cu") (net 1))
 (segment (start 98.09 97.6476) (end 98.09 99.88) (width 1) (layer "F.Cu") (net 1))
 (segment (start 98.09 99.88) (end 99.06 100.85) (width 1) (layer "F.Cu") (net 1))
 (segment (start 96.82 101.31) (end 97.61 102.1) (width 1) (layer "F.Cu") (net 18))
 (segment (start 96.82 97.6476) (end 96.82 101.31) (width 1) (layer "F.Cu") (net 18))
 (segment (start 96.437766 103.42) (end 98.248908 103.42) (width 1) (layer "F.Cu") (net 17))
 (segment (start 98.248908 103.42) (end 100.59 105.761092) (width 1) (layer "F.Cu") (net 17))
 (segment (start 100.59 105.761092) (end 100.59 122.54) (width 1) (layer "F.Cu") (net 17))
 (segment (start 95.55 97.6476) (end 95.55 102.532234) (width 1) (layer "F.Cu") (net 17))
 (segment (start 95.55 102.532234) (end 96.437766 103.42) (width 1) (layer "F.Cu") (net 17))
 (segment (start 98.36 105.298858) (end 98.36 107.32) (width 1) (layer "F.Cu") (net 16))
 (segment (start 94.28 97.6476) (end 94.28 103.03) (width 1) (layer "F.Cu") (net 16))
 (segment (start 98.36 107.32) (end 97.61 108.07) (width 1) (layer "F.Cu") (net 16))
 (segment (start 97.61 108.07) (end 96.91 108.07) (width 1) (layer "F.Cu") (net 16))
 (segment (start 94.28 103.03) (end 95.92 104.67) (width 1) (layer "F.Cu") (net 16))
 (segment (start 95.92 104.67) (end 97.731142 104.67) (width 1) (layer "F.Cu") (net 16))
 (segment (start 97.731142 104.67) (end 98.36 105.298858) (width 1) (layer "F.Cu") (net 16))
 (segment (start 56.89 108.51) (end 70.95 108.51) (width 1) (layer "F.Cu") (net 15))
 (segment (start 91.62 102.31) (end 93.01 100.92) (width 1) (layer "F.Cu") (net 15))
 (segment (start 77.15 102.31) (end 91.62 102.31) (width 1) (layer "F.Cu") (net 15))
 (segment (start 93.01 100.92) (end 93.01 97.6476) (width 1) (layer "F.Cu") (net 15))
 (segment (start 70.95 108.51) (end 77.15 102.31) (width 1) (layer "F.Cu") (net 15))
 (segment (start 95.55 92.72) (end 95.55 90.06) (width 1) (layer "F.Cu") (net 9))
 (segment (start 95.55 90.06) (end 93.92 88.43) (width 1) (layer "F.Cu") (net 9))
 (via (at 93.92 88.43) (size 0.6) (drill 0.3) (layers "F.Cu" "B.Cu") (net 9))
 (segment (start 54.61 101.48) (end 56.35 103.22) (width 1) (layer "B.Cu") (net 9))
 (segment (start 56.35 103.31) (end 56.48 103.44) (width 1) (layer "B.Cu") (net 9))
 (segment (start 93.92 88.43) (end 93.09 87.6) (width 1) (layer "B.Cu") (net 9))
 (segment (start 54.61 89.26) (end 54.61 101.48) (width 1) (layer "B.Cu") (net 9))
 (segment (start 56.48 103.44) (end 61.83 103.44) (width 1) (layer "B.Cu") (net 9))
 (segment (start 56.35 103.22) (end 56.35 103.31) (width 1) (layer "B.Cu") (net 9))
 (segment (start 56.27 87.6) (end 54.61 89.26) (width 1) (layer "B.Cu") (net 9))
 (segment (start 93.09 87.6) (end 56.27 87.6) (width 1) (layer "B.Cu") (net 9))
 (segment (start 62.66 94.56) (end 97.75 94.56) (width 1) (layer "F.Cu") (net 10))
 (segment (start 98.09 94.22) (end 98.09 92.72) (width 1) (layer "F.Cu") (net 10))
 (segment (start 97.75 94.56) (end 98.09 94.22) (width 1) (layer "F.Cu") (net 10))
 (segment (start 61.83 93.73) (end 62.66 94.56) (width 1) (layer "F.Cu") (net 10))
 (segment (start 61.83 92.49) (end 61.83 93.73) (width 1) (layer "F.Cu") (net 10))
 (segment (start 105.655 138.69) (end 105.655 136.125) (width 1) (layer "F.Cu") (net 7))
 (segment (start 105.655 136.125) (end 105.64 136.11) (width 1) (layer "F.Cu") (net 7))
 (segment (start 100.63 97.6476) (end 104.1024 97.6476) (width 1) (layer "F.Cu") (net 7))
 (segment (start 104.1024 97.6476) (end 105.32 96.43) (width 1) (layer "F.Cu") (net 7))
 (via (at 105.32 96.43) (size 0.6) (drill 0.3) (layers "F.Cu" "B.Cu") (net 7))
 (via (at 105.64 136.11) (size 0.6) (drill 0.3) (layers "F.Cu" "B.Cu") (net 7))
 (segment (start 66.34 101.99) (end 68.63 101.99) (width 1) (layer "B.Cu") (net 7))
 (segment (start 105.9 97.01) (end 105.9 106.09) (width 1) (layer "B.Cu") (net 7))
 (segment (start 64.53 100.18) (end 66.34 101.99) (width 1) (layer "B.Cu") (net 7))
 (segment (start 105.64 108.65) (end 104.49 107.5) (width 1) (layer "B.Cu") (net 7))
 (segment (start 70.83 107.5) (end 68.63 105.3) (width 1) (layer "B.Cu") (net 7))
 (segment (start 104.49 107.5) (end 70.83 107.5) (width 1) (layer "B.Cu") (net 7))
 (segment (start 64.53 92.49) (end 64.53 100.18) (width 1) (layer "B.Cu") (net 7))
 (segment (start 105.64 136.11) (end 105.64 108.65) (width 1) (layer "B.Cu") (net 7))
 (segment (start 105.9 106.09) (end 104.49 107.5) (width 1) (layer "B.Cu") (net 7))
 (segment (start 105.32 96.43) (end 105.9 97.01) (width 1) (layer "B.Cu") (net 7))
 (segment (start 68.63 105.3) (end 68.63 101.99) (width 1) (layer "B.Cu") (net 7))
 (segment (start 99.36 92.72) (end 99.36 94.94) (width 1) (layer "F.Cu") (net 6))
 (segment (start 99.36 94.94) (end 98.49 95.81) (width 1) (layer "F.Cu") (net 6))
 (segment (start 98.49 95.81) (end 72.11 95.81) (width 1) (layer "F.Cu") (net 6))
 (segment (start 72.11 95.81) (end 68.63 99.29) (width 1) (layer "F.Cu") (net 6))
 (segment (start 51.815 96.44) (end 51.815 98.495) (width 1) (layer "F.Cu") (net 8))
 (segment (start 52.61 99.29) (end 57.68 99.29) (width 1) (layer "F.Cu") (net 8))
 (segment (start 51.815 98.495) (end 52.61 99.29) (width 1) (layer "F.Cu") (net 8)))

